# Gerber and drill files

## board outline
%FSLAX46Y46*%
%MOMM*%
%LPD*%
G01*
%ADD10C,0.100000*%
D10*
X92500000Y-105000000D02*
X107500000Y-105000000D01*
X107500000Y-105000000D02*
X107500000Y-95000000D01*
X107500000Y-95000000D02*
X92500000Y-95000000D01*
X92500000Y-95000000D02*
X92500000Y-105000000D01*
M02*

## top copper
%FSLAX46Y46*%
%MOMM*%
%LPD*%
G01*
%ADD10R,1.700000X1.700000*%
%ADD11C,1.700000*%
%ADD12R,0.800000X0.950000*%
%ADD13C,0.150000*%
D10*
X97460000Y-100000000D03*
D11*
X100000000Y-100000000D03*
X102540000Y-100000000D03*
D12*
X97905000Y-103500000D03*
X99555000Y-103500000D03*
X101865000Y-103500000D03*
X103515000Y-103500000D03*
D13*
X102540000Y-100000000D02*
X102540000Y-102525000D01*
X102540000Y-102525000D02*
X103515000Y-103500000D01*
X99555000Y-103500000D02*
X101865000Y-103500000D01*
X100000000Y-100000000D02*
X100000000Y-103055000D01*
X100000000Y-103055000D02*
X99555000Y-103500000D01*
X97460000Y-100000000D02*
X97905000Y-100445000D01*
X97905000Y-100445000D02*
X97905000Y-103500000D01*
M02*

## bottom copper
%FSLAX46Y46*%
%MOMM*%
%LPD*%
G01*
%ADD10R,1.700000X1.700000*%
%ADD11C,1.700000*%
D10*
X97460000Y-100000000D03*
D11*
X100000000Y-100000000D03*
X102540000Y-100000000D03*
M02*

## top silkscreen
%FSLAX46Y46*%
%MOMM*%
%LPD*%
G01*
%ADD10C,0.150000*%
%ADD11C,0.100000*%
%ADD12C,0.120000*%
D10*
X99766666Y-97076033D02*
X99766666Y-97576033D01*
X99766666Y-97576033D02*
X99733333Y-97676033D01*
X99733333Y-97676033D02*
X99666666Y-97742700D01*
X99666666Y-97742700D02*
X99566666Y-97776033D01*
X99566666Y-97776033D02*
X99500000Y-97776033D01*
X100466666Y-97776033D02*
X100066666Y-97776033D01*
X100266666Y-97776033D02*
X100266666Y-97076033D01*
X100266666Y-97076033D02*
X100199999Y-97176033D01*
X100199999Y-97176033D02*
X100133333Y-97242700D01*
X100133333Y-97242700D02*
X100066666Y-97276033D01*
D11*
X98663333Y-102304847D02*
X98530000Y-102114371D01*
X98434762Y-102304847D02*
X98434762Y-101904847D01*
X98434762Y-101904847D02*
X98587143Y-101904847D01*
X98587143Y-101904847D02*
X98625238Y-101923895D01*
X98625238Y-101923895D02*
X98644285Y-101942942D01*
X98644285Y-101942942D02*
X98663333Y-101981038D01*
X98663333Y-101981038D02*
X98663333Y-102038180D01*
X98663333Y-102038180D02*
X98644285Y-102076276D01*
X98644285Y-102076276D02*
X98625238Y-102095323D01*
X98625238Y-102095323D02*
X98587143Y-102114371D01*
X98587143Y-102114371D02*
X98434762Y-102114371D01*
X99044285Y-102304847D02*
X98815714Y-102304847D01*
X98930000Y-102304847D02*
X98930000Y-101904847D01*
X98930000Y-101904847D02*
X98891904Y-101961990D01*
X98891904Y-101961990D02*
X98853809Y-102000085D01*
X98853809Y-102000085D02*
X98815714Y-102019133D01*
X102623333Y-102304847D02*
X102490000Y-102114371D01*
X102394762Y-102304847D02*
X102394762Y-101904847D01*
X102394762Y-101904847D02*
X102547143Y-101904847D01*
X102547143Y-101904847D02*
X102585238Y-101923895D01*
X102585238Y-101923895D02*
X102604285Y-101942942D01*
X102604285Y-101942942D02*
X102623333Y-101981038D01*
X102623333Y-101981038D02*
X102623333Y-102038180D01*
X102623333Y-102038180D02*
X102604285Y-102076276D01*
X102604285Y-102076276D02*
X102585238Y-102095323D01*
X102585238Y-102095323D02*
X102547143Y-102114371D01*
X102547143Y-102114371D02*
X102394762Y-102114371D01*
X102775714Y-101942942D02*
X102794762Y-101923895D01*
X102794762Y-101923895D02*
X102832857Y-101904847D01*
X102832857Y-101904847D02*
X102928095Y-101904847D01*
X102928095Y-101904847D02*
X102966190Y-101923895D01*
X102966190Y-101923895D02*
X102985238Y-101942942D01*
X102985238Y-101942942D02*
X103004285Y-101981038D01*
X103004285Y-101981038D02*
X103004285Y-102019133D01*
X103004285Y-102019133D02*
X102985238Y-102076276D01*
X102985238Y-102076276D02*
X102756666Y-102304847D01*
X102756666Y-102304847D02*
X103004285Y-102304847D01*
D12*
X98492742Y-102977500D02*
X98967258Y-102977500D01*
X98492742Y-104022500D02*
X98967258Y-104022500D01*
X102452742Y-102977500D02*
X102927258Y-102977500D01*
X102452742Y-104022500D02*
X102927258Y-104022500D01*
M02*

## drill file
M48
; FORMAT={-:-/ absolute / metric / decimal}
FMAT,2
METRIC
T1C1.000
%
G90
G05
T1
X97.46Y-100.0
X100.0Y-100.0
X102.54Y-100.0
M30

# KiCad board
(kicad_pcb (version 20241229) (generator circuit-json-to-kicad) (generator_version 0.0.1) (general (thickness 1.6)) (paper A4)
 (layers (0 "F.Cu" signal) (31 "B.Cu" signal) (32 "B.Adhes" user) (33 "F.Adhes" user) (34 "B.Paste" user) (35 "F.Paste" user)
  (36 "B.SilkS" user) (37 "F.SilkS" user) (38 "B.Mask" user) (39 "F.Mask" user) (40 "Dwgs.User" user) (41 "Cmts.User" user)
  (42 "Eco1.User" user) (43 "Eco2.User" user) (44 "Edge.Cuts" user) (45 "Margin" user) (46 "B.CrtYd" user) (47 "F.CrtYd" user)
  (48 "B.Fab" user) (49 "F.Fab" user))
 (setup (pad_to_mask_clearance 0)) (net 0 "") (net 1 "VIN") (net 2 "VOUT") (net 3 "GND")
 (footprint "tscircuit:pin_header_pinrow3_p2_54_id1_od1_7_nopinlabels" (layer F.Cu) (at 100 100 0)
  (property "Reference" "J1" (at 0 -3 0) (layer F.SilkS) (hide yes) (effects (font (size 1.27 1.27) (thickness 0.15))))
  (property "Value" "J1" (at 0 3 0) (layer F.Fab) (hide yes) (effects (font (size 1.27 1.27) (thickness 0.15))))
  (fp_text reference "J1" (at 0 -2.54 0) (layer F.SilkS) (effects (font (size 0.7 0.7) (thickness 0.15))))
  (pad "1" thru_hole rect (at -2.54 0 0) (size 1.7 1.7) (drill 1) (layers *.Cu *.Mask) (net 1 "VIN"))
  (pad "2" thru_hole circle (at 0 0 0) (size 1.7 1.7) (drill 1) (layers *.Cu *.Mask) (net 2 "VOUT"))
  (pad "3" thru_hole circle (at 2.54 0 0) (size 1.7 1.7) (drill 1) (layers *.Cu *.Mask) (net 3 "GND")))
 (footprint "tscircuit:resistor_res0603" (layer F.Cu) (at 98.73 103.5 0)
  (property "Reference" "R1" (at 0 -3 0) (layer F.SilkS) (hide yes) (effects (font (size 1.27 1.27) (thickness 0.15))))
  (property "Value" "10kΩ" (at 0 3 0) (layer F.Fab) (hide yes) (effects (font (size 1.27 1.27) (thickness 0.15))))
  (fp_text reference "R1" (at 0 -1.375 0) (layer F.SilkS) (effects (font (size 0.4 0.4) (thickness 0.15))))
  (fp_line (start -0.23725799999999997 -0.5225) (end 0.23725799999999997 -0.5225) (stroke (width 0.12) (type default)) (layer F.SilkS))
  (fp_line (start -0.23725799999999997 0.5225) (end 0.23725799999999997 0.5225) (stroke (width 0.12) (type default)) (layer F.SilkS))
  (pad "1" smd rect (at -0.8250000000000002 0 0) (size 0.8 0.95) (layers F.Cu F.Mask) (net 1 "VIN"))
  (pad "2" smd rect (at 0.825 0 0) (size 0.8 0.95) (layers F.Cu F.Mask) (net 2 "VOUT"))
  (pad "" smd rect (at -0.8250000000000002 0 0) (size 0.5599999999999999 0.6649999999999999) (layers F.Paste))
  (pad "" smd rect (at 0.825 0 0) (size 0.5599999999999999 0.6649999999999999) (layers F.Paste)))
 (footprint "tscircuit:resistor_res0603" (layer F.Cu) (at 102.69 103.5 0)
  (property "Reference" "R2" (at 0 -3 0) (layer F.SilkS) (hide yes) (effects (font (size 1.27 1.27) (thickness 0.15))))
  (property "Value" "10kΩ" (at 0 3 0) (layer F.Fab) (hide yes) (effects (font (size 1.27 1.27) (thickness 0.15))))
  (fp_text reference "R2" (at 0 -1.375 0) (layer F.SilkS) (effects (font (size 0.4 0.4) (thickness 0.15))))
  (fp_line (start -0.2372580000000002 -0.5225) (end 0.2372580000000002 -0.5225) (stroke (width 0.12) (type default)) (layer F.SilkS))
  (fp_line (start -0.2372580000000002 0.5225) (end 0.2372580000000002 0.5225) (stroke (width 0.12) (type default)) (layer F.SilkS))
  (pad "1" smd rect (at -0.825 0 0) (size 0.8 0.95) (layers F.Cu F.Mask) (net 2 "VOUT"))
  (pad "2" smd rect (at 0.8250000000000002 0 0) (size 0.8 0.95) (layers F.Cu F.Mask) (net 3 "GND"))
  (pad "" smd rect (at -0.825 0 0) (size 0.5599999999999999 0.6649999999999999) (layers F.Paste))
  (pad "" smd rect (at 0.8250000000000002 0 0) (size 0.5599999999999999 0.6649999999999999) (layers F.Paste)))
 (segment (start 102.54 100) (end 102.54 102.525) (width 0.15) (layer F.Cu) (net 3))
 (segment (start 102.54 102.525) (end 103.515 103.5) (width 0.15) (layer F.Cu) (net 3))
 (segment (start 99.555 103.5) (end 101.865 103.5) (width 0.15) (layer F.Cu) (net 2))
 (segment (start 100 100) (end 100 103.055) (width 0.15) (layer F.Cu) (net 2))
 (segment (start 100 103.055) (end 99.555 103.5) (width 0.15) (layer F.Cu) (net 2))
 (segment (start 97.46 100) (end 97.905 100.445) (width 0.15) (layer F.Cu) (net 1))
 (segment (start 97.905 100.445) (end 97.905 103.5) (width 0.15) (layer F.Cu) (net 1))
 (gr_line (start 92.5 105) (end 107.5 105) (width 0.1) (layer Edge.Cuts))
 (gr_line (start 107.5 105) (end 107.5 95) (width 0.1) (layer Edge.Cuts))
 (gr_line (start 107.5 95) (end 92.5 95) (width 0.1) (layer Edge.Cuts))
 (gr_line (start 92.5 95) (end 92.5 105) (width 0.1) (layer Edge.Cuts)))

